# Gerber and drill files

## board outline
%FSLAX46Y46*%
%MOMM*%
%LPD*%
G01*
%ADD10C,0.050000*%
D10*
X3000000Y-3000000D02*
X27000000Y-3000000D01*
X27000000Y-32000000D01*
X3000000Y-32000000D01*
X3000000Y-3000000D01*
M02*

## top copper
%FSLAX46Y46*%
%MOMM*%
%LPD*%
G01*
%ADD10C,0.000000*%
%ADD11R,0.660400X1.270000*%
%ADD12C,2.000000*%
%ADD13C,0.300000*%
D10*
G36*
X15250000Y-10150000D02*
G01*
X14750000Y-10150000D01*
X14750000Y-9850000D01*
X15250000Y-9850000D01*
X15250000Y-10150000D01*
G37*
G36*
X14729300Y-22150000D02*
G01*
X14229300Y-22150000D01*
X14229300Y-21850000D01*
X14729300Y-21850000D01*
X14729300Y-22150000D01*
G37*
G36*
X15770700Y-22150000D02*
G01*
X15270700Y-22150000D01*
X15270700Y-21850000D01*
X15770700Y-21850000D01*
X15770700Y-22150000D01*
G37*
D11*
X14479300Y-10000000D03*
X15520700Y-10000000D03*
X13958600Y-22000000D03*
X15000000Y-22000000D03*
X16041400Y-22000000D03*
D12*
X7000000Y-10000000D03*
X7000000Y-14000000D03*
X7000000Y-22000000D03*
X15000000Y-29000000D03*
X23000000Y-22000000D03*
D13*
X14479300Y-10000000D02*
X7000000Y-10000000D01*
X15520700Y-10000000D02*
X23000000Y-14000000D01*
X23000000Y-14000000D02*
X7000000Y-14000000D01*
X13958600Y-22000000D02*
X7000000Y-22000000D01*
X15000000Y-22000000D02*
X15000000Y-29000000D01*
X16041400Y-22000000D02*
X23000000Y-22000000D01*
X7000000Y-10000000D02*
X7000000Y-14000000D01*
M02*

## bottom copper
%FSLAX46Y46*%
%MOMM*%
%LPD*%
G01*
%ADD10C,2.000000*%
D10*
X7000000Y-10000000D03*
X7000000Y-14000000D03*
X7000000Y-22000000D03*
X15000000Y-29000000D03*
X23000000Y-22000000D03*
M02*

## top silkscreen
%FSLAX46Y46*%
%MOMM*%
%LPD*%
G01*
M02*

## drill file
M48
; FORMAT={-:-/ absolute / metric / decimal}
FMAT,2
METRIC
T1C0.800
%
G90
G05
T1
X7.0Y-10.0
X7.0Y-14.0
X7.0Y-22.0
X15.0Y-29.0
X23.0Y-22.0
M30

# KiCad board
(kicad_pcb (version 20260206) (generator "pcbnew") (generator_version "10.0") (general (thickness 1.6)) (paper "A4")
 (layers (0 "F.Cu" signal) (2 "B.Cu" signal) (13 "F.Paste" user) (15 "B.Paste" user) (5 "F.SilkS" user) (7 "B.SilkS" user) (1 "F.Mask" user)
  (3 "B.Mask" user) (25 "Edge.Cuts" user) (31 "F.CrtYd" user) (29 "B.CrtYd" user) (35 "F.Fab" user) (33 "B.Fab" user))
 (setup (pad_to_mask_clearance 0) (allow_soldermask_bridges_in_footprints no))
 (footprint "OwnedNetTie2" (layer "F.Cu") (at 15 10)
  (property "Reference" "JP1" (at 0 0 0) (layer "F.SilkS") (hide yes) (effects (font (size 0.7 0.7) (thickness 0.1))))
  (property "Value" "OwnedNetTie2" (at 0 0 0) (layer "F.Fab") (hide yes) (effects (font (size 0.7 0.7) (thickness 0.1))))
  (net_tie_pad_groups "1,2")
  (fp_poly (pts (xy -0.25 -0.15) (xy 0.25 -0.15) (xy 0.25 0.15) (xy -0.25 0.15)) (stroke (width 0) (type solid)) (fill yes) (layer "F.Cu"))
  (pad "1" smd rect (at -0.5207 0) (size 0.6604 1.27) (layers "F.Cu" "F.Mask") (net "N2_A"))
  (pad "2" smd rect (at 0.5207 0) (size 0.6604 1.27) (layers "F.Cu" "F.Mask") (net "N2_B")))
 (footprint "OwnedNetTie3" (layer "F.Cu") (at 15 22)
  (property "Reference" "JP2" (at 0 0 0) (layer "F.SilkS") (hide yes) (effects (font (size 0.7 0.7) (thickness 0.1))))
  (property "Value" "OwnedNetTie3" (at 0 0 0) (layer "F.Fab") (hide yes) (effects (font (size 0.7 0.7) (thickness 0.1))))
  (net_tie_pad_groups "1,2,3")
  (fp_poly
   (pts (xy -0.7707 -0.15) (xy -0.2707 -0.15) (xy -0.2707 0.15) (xy -0.7707 0.15)) (stroke (width 0) (type solid)) (fill yes) (layer "F.Cu"))
  (fp_poly
   (pts (xy 0.2707 -0.15) (xy 0.7707 -0.15) (xy 0.7707 0.15) (xy 0.2707 0.15)) (stroke (width 0) (type solid)) (fill yes) (layer "F.Cu"))
  (pad "1" smd rect (at -1.0414 0) (size 0.6604 1.27) (layers "F.Cu" "F.Mask") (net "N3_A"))
  (pad "2" smd rect (at 0 0) (size 0.6604 1.27) (layers "F.Cu" "F.Mask") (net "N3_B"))
  (pad "3" smd rect (at 1.0414 0) (size 0.6604 1.27) (layers "F.Cu" "F.Mask") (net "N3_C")))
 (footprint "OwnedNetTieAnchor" (layer "F.Cu") (at 7 10)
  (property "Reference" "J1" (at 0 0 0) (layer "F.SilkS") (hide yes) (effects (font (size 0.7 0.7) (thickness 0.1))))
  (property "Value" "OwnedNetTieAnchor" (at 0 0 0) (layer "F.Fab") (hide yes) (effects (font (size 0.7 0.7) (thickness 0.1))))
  (pad "1" thru_hole circle (at 0 0) (size 2 2) (drill 0.8) (layers "*.Cu" "*.Mask") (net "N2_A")))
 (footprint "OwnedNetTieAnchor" (layer "F.Cu") (at 7 14)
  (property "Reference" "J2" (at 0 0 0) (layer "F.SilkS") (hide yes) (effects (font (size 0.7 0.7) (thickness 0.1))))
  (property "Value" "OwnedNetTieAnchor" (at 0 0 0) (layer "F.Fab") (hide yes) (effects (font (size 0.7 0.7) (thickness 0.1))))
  (pad "1" thru_hole circle (at 0 0) (size 2 2) (drill 0.8) (layers "*.Cu" "*.Mask") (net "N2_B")))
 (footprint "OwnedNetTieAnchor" (layer "F.Cu") (at 7 22)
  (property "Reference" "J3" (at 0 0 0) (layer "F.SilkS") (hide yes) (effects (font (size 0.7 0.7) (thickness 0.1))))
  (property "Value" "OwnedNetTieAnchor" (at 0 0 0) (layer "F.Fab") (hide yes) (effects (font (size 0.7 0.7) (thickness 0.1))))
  (pad "1" thru_hole circle (at 0 0) (size 2 2) (drill 0.8) (layers "*.Cu" "*.Mask") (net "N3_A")))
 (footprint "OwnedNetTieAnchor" (layer "F.Cu") (at 15 29)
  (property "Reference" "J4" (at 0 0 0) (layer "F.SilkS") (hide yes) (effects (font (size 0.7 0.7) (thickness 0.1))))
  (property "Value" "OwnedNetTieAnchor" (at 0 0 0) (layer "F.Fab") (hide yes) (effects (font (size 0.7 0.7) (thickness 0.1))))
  (pad "1" thru_hole circle (at 0 0) (size 2 2) (drill 0.8) (layers "*.Cu" "*.Mask") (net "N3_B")))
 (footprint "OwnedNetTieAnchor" (layer "F.Cu") (at 23 22)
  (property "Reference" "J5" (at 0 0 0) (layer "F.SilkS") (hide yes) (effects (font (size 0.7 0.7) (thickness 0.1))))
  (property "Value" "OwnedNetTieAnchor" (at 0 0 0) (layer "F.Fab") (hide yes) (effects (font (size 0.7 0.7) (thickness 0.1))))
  (pad "1" thru_hole circle (at 0 0) (size 2 2) (drill 0.8) (layers "*.Cu" "*.Mask") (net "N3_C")))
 (segment (start 14.4793 10) (end 7 10) (width 0.3) (layer "F.Cu") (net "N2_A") (locked yes))
 (segment (start 15.5207 10) (end 23 14) (width 0.3) (layer "F.Cu") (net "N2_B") (locked yes))
 (segment (start 23 14) (end 7 14) (width 0.3) (layer "F.Cu") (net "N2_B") (locked yes))
 (segment (start 13.9586 22) (end 7 22) (width 0.3) (layer "F.Cu") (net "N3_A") (locked yes))
 (segment (start 15 22) (end 15 29) (width 0.3) (layer "F.Cu") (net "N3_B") (locked yes))
 (segment (start 16.0414 22) (end 23 22) (width 0.3) (layer "F.Cu") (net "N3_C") (locked yes))
 (gr_rect (start 3 3) (end 27 32) (stroke (width 0.05) (type default)) (fill none) (layer "Edge.Cuts"))
 (segment (start 7 10) (end 7 14) (width 0.3) (layer "F.Cu") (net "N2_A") (locked yes)))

